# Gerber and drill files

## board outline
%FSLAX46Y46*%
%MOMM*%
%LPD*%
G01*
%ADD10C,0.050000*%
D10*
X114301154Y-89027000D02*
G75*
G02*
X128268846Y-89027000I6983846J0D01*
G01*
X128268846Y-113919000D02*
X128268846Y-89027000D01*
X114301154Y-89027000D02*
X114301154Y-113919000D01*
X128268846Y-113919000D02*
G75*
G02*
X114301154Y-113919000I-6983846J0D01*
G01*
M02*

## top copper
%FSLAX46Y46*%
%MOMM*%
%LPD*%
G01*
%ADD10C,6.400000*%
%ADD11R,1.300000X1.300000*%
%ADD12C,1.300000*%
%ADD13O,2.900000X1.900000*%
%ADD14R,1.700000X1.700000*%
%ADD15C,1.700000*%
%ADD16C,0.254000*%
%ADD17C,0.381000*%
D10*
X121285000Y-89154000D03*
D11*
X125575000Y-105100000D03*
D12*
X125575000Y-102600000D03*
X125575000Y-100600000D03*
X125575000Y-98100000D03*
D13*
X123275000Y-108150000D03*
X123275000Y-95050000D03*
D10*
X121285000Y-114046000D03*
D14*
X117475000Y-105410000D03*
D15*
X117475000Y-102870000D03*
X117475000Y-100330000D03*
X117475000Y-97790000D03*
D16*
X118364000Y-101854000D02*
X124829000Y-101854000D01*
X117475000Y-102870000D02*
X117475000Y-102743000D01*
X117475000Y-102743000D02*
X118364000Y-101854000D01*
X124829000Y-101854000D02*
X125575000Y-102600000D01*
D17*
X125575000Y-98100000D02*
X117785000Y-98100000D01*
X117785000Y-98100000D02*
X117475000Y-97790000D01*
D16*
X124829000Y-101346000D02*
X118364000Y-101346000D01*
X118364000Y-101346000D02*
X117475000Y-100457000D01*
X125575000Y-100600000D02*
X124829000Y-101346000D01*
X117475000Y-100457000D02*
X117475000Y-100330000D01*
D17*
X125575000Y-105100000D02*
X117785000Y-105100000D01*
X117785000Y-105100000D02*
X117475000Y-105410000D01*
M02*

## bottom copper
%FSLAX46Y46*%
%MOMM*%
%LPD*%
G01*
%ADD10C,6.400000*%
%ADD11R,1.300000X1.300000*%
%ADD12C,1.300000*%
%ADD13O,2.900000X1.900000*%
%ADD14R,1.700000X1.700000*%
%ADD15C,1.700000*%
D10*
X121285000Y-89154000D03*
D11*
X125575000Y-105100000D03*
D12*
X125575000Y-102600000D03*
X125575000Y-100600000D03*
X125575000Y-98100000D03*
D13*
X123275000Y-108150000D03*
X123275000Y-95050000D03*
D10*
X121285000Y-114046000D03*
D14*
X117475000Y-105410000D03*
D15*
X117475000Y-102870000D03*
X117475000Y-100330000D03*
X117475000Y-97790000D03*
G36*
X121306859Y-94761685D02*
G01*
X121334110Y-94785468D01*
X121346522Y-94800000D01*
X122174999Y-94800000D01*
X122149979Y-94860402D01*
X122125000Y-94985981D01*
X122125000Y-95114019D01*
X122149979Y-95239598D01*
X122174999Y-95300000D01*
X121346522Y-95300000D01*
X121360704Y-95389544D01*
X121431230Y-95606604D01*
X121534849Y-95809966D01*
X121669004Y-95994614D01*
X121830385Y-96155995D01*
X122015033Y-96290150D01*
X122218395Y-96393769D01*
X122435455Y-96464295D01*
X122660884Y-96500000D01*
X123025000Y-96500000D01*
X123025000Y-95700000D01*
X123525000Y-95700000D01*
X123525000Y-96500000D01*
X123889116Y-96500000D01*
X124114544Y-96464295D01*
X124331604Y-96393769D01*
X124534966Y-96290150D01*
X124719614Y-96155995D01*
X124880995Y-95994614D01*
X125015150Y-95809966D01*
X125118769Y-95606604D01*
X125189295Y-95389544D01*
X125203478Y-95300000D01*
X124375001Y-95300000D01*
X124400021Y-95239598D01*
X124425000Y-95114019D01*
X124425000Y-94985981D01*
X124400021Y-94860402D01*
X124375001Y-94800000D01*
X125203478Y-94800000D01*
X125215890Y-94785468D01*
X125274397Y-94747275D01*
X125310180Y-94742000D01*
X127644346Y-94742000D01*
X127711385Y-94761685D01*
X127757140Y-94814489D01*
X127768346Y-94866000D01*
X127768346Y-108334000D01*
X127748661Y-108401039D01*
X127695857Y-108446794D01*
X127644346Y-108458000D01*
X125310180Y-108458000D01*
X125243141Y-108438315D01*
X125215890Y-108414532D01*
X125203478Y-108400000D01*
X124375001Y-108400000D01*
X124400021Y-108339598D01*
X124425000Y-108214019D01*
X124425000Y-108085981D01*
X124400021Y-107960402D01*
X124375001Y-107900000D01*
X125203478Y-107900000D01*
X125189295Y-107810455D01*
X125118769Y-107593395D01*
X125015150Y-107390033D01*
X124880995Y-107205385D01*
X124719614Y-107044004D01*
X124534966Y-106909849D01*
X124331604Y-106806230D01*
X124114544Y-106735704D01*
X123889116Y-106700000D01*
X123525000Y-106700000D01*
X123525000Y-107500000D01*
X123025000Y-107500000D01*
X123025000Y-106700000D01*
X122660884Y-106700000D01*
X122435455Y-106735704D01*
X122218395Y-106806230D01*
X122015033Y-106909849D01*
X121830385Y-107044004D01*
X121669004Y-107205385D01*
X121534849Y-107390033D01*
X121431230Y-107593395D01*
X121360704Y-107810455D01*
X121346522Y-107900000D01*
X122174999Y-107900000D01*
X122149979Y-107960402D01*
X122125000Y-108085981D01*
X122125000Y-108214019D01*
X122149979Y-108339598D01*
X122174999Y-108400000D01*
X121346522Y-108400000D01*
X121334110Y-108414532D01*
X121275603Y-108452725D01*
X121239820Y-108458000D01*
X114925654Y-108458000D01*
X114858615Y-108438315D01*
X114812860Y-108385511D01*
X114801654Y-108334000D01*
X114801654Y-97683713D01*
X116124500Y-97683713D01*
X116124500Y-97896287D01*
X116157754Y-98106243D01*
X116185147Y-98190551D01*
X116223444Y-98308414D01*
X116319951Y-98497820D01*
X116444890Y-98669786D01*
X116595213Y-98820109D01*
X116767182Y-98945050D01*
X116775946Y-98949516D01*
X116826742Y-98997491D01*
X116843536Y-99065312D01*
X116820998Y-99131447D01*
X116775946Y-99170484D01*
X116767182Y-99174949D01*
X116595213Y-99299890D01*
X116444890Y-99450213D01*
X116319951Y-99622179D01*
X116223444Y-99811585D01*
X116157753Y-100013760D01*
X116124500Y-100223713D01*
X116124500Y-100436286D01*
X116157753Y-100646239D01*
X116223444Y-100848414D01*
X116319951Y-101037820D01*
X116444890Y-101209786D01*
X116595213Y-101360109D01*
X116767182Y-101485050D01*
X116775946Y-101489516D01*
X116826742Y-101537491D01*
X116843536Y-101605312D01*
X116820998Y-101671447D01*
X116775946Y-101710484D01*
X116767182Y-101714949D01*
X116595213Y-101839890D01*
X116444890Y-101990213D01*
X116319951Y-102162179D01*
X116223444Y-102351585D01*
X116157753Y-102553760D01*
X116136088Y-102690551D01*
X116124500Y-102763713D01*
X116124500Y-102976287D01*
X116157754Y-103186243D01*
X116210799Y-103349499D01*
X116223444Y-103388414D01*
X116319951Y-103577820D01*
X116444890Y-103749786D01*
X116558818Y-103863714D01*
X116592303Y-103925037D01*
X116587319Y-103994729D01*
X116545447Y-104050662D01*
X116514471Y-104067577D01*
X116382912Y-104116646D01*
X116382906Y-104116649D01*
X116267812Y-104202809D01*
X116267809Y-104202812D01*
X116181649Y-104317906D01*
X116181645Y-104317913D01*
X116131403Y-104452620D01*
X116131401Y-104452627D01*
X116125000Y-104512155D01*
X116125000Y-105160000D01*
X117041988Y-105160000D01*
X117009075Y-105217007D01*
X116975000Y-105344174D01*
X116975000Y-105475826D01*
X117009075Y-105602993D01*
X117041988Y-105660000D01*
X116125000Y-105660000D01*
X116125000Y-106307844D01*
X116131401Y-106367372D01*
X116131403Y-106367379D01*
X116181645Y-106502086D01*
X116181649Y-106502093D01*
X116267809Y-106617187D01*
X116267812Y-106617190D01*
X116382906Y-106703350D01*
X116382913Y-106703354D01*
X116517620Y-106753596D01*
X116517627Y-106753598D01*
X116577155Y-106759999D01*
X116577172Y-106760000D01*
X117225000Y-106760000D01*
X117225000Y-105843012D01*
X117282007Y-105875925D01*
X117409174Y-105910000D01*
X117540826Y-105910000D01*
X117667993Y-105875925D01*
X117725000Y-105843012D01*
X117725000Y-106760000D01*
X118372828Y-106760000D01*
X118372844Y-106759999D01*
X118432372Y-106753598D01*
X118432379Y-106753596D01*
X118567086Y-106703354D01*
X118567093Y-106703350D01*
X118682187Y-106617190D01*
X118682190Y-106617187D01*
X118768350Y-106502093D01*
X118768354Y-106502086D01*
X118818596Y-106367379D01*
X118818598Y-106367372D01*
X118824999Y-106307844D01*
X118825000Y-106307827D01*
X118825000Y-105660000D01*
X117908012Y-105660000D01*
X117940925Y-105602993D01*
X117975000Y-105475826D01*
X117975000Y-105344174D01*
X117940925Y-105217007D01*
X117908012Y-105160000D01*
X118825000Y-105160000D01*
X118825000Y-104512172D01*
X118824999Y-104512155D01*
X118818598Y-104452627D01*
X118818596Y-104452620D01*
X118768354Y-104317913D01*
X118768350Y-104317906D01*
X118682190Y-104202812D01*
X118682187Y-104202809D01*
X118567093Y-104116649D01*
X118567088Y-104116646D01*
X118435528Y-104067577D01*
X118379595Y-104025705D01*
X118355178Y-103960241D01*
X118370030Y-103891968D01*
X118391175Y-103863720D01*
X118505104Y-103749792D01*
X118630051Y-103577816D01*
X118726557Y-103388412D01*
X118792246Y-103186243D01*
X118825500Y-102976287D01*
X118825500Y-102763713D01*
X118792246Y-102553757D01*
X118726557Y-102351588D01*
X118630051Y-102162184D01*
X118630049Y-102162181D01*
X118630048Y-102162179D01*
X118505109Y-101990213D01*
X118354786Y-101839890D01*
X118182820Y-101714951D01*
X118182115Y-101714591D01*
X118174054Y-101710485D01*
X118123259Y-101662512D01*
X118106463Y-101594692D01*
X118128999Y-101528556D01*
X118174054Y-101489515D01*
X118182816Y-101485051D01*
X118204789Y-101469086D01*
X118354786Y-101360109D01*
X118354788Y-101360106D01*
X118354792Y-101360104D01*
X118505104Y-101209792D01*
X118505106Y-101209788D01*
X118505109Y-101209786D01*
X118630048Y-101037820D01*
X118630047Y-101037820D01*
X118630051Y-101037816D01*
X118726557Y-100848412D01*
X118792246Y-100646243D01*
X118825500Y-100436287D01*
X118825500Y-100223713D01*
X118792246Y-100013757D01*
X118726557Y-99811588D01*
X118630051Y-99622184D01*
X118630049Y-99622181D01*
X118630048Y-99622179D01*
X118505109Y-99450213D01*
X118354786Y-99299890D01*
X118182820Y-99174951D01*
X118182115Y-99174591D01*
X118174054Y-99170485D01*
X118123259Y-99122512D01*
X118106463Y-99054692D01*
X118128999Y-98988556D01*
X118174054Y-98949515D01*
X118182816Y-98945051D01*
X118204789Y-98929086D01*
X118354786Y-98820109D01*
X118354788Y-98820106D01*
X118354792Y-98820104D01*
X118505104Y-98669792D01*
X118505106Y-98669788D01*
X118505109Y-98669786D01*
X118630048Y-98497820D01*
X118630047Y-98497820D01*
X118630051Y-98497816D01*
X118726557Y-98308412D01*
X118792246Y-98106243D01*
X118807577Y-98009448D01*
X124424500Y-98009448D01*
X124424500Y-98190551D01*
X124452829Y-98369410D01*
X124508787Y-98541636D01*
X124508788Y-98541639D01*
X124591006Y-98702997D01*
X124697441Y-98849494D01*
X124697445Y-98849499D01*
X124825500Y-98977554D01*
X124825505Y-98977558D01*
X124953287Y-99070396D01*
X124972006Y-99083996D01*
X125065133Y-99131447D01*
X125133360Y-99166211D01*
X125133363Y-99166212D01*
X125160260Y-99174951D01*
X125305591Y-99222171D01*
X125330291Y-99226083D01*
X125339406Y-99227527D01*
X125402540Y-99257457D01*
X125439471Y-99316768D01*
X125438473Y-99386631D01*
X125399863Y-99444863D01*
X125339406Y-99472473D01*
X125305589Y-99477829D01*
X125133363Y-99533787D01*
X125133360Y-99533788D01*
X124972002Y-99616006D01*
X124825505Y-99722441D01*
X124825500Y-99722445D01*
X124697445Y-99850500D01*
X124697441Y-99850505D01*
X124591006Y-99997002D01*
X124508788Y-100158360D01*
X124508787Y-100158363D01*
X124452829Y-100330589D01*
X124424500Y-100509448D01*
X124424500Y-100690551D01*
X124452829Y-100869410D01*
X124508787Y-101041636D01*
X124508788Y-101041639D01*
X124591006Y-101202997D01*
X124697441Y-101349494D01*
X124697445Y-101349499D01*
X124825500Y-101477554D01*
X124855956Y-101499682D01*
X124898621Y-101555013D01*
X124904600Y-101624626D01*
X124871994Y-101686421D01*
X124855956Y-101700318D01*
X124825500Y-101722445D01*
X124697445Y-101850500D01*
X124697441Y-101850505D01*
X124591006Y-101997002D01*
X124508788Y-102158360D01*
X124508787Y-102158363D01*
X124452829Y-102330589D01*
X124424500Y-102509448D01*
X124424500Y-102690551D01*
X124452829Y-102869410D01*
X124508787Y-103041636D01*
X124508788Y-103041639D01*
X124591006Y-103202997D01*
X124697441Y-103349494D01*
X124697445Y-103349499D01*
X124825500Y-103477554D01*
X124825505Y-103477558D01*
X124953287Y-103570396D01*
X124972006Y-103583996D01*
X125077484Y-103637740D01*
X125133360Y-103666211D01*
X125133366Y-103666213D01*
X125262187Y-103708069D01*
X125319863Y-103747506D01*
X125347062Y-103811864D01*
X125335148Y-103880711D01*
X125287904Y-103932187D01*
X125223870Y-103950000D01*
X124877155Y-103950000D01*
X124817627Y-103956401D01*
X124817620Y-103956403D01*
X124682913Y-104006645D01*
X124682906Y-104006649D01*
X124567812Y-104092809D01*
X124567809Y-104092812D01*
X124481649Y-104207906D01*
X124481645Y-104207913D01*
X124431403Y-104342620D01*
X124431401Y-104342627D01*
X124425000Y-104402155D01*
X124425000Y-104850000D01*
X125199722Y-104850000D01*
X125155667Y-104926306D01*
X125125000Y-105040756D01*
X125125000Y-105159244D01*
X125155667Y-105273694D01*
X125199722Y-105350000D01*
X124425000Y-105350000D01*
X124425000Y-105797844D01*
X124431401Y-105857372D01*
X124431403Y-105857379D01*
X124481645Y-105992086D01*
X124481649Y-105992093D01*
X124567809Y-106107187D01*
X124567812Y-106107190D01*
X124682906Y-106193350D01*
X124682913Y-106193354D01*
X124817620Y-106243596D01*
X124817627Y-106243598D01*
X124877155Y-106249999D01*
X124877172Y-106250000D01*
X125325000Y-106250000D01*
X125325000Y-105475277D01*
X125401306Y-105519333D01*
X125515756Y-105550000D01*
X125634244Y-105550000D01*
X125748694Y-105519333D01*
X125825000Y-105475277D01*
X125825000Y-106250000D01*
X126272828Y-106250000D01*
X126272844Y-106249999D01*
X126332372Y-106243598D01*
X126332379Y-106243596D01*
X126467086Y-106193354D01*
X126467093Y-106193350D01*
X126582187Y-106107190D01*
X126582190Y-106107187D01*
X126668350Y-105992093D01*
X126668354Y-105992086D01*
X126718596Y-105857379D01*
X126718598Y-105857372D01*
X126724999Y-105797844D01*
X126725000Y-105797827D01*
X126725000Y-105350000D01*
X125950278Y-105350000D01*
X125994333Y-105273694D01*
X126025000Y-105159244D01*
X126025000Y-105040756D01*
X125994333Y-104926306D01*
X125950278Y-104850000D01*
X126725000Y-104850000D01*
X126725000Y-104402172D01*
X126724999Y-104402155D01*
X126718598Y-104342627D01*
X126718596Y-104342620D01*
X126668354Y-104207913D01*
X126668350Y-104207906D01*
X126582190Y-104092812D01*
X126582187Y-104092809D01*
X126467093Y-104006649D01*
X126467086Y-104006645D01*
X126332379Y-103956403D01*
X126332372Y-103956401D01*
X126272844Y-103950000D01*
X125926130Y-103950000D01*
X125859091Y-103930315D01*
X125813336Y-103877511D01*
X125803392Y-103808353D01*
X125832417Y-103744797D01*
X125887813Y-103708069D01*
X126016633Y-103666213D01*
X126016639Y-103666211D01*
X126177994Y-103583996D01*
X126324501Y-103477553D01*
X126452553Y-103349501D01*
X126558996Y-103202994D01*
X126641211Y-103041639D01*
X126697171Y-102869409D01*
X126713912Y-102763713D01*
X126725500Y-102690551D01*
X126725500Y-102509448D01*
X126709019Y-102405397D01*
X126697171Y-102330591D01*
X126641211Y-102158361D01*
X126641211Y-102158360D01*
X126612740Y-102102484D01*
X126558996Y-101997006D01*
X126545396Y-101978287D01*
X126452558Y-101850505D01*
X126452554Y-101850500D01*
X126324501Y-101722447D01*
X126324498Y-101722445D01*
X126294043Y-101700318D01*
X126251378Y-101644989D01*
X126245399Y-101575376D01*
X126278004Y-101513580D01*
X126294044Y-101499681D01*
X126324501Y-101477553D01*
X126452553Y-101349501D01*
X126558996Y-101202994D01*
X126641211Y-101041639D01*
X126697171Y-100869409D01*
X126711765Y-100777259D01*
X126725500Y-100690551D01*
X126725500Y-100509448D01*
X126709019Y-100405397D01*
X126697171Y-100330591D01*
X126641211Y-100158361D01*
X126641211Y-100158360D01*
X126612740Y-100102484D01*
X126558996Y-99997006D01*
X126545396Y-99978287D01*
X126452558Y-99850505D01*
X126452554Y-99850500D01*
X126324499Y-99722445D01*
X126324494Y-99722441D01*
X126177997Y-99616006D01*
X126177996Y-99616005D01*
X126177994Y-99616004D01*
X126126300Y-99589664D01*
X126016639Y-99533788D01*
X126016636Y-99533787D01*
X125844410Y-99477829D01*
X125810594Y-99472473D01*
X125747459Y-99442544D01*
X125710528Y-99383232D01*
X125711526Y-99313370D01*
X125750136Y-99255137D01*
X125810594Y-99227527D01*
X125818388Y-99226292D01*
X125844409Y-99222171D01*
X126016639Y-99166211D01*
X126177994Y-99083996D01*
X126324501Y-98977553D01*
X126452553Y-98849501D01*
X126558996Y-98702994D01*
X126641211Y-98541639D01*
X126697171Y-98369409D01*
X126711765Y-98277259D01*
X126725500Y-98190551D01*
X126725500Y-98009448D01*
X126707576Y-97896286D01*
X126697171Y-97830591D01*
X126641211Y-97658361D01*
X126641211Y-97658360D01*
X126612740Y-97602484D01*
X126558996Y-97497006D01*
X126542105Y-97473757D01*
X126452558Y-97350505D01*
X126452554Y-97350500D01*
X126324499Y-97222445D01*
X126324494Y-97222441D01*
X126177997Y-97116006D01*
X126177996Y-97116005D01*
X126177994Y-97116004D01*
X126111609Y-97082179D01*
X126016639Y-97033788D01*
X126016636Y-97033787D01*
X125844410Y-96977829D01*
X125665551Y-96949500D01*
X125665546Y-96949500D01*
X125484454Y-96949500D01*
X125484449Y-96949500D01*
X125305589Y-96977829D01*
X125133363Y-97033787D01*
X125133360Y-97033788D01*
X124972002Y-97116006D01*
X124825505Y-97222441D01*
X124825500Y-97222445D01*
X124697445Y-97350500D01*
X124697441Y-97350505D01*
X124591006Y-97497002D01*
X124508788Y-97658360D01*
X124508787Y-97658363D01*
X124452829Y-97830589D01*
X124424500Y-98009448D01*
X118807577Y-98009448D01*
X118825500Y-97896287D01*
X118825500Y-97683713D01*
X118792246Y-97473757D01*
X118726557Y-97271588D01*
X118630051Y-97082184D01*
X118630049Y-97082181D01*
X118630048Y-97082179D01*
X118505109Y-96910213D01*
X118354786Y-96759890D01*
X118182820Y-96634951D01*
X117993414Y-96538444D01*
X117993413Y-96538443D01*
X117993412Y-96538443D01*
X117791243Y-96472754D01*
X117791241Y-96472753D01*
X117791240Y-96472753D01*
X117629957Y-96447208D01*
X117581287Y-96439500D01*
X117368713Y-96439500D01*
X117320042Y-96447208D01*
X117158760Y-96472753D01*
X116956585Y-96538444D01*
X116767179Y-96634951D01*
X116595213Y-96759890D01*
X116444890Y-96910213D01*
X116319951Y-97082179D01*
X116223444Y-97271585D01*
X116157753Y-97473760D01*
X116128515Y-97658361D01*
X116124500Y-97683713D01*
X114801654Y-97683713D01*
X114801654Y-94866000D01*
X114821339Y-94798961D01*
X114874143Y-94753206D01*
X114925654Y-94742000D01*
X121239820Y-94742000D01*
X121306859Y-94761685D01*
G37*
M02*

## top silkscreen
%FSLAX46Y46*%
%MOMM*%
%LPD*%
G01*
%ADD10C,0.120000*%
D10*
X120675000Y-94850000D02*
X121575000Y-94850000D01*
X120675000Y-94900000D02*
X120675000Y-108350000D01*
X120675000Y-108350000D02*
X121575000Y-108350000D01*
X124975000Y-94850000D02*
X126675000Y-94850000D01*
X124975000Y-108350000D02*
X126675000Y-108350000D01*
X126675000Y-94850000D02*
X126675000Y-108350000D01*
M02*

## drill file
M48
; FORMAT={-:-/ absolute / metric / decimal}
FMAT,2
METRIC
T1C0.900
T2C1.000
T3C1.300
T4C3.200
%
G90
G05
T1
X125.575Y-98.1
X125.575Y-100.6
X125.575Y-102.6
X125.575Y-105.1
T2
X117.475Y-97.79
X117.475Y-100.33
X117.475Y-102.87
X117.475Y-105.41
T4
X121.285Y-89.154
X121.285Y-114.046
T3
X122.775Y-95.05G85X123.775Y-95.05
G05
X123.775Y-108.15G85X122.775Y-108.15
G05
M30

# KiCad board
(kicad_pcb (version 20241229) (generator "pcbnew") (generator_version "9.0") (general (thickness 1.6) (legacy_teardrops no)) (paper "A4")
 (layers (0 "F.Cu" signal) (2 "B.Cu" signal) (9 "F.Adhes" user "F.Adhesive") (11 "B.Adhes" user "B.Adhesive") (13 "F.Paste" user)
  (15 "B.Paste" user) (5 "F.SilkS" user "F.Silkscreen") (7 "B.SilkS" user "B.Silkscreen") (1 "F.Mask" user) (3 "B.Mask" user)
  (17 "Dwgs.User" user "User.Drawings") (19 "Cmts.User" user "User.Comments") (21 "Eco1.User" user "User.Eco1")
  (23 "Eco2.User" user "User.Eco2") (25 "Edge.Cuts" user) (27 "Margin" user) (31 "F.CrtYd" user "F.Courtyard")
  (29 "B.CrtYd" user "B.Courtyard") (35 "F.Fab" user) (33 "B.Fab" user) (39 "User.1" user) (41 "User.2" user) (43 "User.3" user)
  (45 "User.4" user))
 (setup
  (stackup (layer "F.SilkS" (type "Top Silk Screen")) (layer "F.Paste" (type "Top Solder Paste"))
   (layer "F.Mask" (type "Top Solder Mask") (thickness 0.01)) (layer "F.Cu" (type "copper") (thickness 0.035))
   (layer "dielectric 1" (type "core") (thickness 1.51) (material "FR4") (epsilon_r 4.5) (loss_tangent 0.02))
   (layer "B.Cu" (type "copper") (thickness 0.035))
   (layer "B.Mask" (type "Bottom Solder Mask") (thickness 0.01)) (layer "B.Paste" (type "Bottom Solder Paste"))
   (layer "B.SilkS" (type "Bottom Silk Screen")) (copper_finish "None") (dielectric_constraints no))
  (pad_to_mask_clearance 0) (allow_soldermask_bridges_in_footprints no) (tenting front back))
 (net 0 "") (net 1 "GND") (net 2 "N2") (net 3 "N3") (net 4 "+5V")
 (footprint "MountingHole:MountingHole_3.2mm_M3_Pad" (layer "F.Cu") (at 121.285 89.154)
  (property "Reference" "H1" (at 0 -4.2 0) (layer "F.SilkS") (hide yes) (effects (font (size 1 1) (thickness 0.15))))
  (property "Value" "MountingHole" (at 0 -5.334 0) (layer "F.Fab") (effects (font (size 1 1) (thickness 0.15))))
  (pad "1" thru_hole circle (at 0 0) (size 6.4 6.4) (drill 3.2) (layers "*.Cu" "*.Mask") (remove_unused_layers no)))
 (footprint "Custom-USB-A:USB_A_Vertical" (layer "F.Cu") (at 125.575 105.1 90)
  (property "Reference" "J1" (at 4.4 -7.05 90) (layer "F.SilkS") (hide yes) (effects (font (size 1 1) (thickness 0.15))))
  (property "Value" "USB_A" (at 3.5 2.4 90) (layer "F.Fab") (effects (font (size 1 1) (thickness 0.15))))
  (fp_line (start 10.25 -4.9) (end 10.25 -4) (stroke (width 0.12) (type solid)) (layer "F.SilkS"))
  (fp_line (start 10.2 -4.9) (end -3.25 -4.9) (stroke (width 0.12) (type solid)) (layer "F.SilkS"))
  (fp_line (start -3.25 -4.9) (end -3.25 -4) (stroke (width 0.12) (type solid)) (layer "F.SilkS"))
  (fp_line (start 10.25 -0.6) (end 10.25 1.1) (stroke (width 0.12) (type solid)) (layer "F.SilkS"))
  (fp_line (start -3.25 -0.6) (end -3.25 1.1) (stroke (width 0.12) (type solid)) (layer "F.SilkS"))
  (fp_line (start 10.25 1.1) (end -3.25 1.1) (stroke (width 0.12) (type solid)) (layer "F.SilkS"))
  (pad "1" thru_hole rect (at 0 0 90) (size 1.3 1.3) (drill 0.9) (layers "*.Cu" "*.Mask") (remove_unused_layers no) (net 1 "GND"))
  (pad "2" thru_hole circle (at 2.5 0 90) (size 1.3 1.3) (drill 0.9) (layers "*.Cu" "*.Mask") (remove_unused_layers no) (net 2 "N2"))
  (pad "3" thru_hole circle (at 4.5 0 90) (size 1.3 1.3) (drill 0.9) (layers "*.Cu" "*.Mask") (remove_unused_layers no) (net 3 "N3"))
  (pad "4" thru_hole circle (at 7 0 90) (size 1.3 1.3) (drill 0.9) (layers "*.Cu" "*.Mask") (remove_unused_layers no) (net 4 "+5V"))
  (pad "5" thru_hole oval (at -3.05 -2.3 270) (size 1.9 2.9) (drill oval 1.3 2.3) (layers "*.Cu" "*.Mask") (remove_unused_layers no)
   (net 1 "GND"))
  (pad "5" thru_hole oval (at 10.05 -2.3 90) (size 1.9 2.9) (drill oval 1.3 2.3) (layers "*.Cu" "*.Mask") (remove_unused_layers no)
   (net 1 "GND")))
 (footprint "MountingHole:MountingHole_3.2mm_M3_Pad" (layer "F.Cu") (at 121.285 114.046)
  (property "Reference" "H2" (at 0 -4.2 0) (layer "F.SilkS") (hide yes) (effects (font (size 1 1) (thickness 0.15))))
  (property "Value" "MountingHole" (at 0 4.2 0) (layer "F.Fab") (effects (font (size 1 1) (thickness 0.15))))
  (pad "1" thru_hole circle (at 0 0) (size 6.4 6.4) (drill 3.2) (layers "*.Cu" "*.Mask") (remove_unused_layers no)))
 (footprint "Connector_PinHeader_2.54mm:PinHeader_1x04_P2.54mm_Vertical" (layer "B.Cu") (at 117.475 105.41)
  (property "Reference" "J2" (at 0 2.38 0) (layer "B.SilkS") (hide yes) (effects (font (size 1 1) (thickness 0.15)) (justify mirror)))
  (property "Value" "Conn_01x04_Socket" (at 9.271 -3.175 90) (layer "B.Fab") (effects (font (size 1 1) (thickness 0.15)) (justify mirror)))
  (pad "1" thru_hole rect (at 0 0) (size 1.7 1.7) (drill 1) (layers "*.Cu" "*.Mask") (remove_unused_layers no) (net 1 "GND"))
  (pad "2" thru_hole circle (at 0 -2.54) (size 1.7 1.7) (drill 1) (layers "*.Cu" "*.Mask") (remove_unused_layers no) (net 2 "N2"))
  (pad "3" thru_hole circle (at 0 -5.08) (size 1.7 1.7) (drill 1) (layers "*.Cu" "*.Mask") (remove_unused_layers no) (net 3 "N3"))
  (pad "4" thru_hole circle (at 0 -7.62) (size 1.7 1.7) (drill 1) (layers "*.Cu" "*.Mask") (remove_unused_layers no) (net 4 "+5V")))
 (gr_arc (start 114.301154 89.027) (mid 121.285 82.043154) (end 128.268846 89.027) (stroke (width 0.05) (type default)) (layer "Edge.Cuts"))
 (gr_line (start 128.268846 113.919) (end 128.268846 89.027) (stroke (width 0.05) (type default)) (layer "Edge.Cuts"))
 (gr_line (start 114.301154 89.027) (end 114.301154 113.919) (stroke (width 0.05) (type default)) (layer "Edge.Cuts"))
 (gr_arc (start 128.268846 113.919) (mid 121.285 120.902846) (end 114.301154 113.919) (stroke (width 0.05) (type default))
  (layer "Edge.Cuts"))
 (segment (start 118.364 101.854) (end 124.829 101.854) (width 0.254) (layer "F.Cu") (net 2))
 (segment (start 117.475 102.87) (end 117.475 102.743) (width 0.254) (layer "F.Cu") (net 2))
 (segment (start 117.475 102.743) (end 118.364 101.854) (width 0.254) (layer "F.Cu") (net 2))
 (segment (start 124.829 101.854) (end 125.575 102.6) (width 0.254) (layer "F.Cu") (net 2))
 (segment (start 125.575 98.1) (end 117.785 98.1) (width 0.381) (layer "F.Cu") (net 4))
 (segment (start 117.785 98.1) (end 117.475 97.79) (width 0.381) (layer "F.Cu") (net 4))
 (segment (start 124.829 101.346) (end 118.364 101.346) (width 0.254) (layer "F.Cu") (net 3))
 (segment (start 118.364 101.346) (end 117.475 100.457) (width 0.254) (layer "F.Cu") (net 3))
 (segment (start 125.575 100.6) (end 124.829 101.346) (width 0.254) (layer "F.Cu") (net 3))
 (segment (start 117.475 100.457) (end 117.475 100.33) (width 0.254) (layer "F.Cu") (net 3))
 (segment (start 125.575 105.1) (end 117.785 105.1) (width 0.381) (layer "F.Cu") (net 1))
 (segment (start 117.785 105.1) (end 117.475 105.41) (width 0.381) (layer "F.Cu") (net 1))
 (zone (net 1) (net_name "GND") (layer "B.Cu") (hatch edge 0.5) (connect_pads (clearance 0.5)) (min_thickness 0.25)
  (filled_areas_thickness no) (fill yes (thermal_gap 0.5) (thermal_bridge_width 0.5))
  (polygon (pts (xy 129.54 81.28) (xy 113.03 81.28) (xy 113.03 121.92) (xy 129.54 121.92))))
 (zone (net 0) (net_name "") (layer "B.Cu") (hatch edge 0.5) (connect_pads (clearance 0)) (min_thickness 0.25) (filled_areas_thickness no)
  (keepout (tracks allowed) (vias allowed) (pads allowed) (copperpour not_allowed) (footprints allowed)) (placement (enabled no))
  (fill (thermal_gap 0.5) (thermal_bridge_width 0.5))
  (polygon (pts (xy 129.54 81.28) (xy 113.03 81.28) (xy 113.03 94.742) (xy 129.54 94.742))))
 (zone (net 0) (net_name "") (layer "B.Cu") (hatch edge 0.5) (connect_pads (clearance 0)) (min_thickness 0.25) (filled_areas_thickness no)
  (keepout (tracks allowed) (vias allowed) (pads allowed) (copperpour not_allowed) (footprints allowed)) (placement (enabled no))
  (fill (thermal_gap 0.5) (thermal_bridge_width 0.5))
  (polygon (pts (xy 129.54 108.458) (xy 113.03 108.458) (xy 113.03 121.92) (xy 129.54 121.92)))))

